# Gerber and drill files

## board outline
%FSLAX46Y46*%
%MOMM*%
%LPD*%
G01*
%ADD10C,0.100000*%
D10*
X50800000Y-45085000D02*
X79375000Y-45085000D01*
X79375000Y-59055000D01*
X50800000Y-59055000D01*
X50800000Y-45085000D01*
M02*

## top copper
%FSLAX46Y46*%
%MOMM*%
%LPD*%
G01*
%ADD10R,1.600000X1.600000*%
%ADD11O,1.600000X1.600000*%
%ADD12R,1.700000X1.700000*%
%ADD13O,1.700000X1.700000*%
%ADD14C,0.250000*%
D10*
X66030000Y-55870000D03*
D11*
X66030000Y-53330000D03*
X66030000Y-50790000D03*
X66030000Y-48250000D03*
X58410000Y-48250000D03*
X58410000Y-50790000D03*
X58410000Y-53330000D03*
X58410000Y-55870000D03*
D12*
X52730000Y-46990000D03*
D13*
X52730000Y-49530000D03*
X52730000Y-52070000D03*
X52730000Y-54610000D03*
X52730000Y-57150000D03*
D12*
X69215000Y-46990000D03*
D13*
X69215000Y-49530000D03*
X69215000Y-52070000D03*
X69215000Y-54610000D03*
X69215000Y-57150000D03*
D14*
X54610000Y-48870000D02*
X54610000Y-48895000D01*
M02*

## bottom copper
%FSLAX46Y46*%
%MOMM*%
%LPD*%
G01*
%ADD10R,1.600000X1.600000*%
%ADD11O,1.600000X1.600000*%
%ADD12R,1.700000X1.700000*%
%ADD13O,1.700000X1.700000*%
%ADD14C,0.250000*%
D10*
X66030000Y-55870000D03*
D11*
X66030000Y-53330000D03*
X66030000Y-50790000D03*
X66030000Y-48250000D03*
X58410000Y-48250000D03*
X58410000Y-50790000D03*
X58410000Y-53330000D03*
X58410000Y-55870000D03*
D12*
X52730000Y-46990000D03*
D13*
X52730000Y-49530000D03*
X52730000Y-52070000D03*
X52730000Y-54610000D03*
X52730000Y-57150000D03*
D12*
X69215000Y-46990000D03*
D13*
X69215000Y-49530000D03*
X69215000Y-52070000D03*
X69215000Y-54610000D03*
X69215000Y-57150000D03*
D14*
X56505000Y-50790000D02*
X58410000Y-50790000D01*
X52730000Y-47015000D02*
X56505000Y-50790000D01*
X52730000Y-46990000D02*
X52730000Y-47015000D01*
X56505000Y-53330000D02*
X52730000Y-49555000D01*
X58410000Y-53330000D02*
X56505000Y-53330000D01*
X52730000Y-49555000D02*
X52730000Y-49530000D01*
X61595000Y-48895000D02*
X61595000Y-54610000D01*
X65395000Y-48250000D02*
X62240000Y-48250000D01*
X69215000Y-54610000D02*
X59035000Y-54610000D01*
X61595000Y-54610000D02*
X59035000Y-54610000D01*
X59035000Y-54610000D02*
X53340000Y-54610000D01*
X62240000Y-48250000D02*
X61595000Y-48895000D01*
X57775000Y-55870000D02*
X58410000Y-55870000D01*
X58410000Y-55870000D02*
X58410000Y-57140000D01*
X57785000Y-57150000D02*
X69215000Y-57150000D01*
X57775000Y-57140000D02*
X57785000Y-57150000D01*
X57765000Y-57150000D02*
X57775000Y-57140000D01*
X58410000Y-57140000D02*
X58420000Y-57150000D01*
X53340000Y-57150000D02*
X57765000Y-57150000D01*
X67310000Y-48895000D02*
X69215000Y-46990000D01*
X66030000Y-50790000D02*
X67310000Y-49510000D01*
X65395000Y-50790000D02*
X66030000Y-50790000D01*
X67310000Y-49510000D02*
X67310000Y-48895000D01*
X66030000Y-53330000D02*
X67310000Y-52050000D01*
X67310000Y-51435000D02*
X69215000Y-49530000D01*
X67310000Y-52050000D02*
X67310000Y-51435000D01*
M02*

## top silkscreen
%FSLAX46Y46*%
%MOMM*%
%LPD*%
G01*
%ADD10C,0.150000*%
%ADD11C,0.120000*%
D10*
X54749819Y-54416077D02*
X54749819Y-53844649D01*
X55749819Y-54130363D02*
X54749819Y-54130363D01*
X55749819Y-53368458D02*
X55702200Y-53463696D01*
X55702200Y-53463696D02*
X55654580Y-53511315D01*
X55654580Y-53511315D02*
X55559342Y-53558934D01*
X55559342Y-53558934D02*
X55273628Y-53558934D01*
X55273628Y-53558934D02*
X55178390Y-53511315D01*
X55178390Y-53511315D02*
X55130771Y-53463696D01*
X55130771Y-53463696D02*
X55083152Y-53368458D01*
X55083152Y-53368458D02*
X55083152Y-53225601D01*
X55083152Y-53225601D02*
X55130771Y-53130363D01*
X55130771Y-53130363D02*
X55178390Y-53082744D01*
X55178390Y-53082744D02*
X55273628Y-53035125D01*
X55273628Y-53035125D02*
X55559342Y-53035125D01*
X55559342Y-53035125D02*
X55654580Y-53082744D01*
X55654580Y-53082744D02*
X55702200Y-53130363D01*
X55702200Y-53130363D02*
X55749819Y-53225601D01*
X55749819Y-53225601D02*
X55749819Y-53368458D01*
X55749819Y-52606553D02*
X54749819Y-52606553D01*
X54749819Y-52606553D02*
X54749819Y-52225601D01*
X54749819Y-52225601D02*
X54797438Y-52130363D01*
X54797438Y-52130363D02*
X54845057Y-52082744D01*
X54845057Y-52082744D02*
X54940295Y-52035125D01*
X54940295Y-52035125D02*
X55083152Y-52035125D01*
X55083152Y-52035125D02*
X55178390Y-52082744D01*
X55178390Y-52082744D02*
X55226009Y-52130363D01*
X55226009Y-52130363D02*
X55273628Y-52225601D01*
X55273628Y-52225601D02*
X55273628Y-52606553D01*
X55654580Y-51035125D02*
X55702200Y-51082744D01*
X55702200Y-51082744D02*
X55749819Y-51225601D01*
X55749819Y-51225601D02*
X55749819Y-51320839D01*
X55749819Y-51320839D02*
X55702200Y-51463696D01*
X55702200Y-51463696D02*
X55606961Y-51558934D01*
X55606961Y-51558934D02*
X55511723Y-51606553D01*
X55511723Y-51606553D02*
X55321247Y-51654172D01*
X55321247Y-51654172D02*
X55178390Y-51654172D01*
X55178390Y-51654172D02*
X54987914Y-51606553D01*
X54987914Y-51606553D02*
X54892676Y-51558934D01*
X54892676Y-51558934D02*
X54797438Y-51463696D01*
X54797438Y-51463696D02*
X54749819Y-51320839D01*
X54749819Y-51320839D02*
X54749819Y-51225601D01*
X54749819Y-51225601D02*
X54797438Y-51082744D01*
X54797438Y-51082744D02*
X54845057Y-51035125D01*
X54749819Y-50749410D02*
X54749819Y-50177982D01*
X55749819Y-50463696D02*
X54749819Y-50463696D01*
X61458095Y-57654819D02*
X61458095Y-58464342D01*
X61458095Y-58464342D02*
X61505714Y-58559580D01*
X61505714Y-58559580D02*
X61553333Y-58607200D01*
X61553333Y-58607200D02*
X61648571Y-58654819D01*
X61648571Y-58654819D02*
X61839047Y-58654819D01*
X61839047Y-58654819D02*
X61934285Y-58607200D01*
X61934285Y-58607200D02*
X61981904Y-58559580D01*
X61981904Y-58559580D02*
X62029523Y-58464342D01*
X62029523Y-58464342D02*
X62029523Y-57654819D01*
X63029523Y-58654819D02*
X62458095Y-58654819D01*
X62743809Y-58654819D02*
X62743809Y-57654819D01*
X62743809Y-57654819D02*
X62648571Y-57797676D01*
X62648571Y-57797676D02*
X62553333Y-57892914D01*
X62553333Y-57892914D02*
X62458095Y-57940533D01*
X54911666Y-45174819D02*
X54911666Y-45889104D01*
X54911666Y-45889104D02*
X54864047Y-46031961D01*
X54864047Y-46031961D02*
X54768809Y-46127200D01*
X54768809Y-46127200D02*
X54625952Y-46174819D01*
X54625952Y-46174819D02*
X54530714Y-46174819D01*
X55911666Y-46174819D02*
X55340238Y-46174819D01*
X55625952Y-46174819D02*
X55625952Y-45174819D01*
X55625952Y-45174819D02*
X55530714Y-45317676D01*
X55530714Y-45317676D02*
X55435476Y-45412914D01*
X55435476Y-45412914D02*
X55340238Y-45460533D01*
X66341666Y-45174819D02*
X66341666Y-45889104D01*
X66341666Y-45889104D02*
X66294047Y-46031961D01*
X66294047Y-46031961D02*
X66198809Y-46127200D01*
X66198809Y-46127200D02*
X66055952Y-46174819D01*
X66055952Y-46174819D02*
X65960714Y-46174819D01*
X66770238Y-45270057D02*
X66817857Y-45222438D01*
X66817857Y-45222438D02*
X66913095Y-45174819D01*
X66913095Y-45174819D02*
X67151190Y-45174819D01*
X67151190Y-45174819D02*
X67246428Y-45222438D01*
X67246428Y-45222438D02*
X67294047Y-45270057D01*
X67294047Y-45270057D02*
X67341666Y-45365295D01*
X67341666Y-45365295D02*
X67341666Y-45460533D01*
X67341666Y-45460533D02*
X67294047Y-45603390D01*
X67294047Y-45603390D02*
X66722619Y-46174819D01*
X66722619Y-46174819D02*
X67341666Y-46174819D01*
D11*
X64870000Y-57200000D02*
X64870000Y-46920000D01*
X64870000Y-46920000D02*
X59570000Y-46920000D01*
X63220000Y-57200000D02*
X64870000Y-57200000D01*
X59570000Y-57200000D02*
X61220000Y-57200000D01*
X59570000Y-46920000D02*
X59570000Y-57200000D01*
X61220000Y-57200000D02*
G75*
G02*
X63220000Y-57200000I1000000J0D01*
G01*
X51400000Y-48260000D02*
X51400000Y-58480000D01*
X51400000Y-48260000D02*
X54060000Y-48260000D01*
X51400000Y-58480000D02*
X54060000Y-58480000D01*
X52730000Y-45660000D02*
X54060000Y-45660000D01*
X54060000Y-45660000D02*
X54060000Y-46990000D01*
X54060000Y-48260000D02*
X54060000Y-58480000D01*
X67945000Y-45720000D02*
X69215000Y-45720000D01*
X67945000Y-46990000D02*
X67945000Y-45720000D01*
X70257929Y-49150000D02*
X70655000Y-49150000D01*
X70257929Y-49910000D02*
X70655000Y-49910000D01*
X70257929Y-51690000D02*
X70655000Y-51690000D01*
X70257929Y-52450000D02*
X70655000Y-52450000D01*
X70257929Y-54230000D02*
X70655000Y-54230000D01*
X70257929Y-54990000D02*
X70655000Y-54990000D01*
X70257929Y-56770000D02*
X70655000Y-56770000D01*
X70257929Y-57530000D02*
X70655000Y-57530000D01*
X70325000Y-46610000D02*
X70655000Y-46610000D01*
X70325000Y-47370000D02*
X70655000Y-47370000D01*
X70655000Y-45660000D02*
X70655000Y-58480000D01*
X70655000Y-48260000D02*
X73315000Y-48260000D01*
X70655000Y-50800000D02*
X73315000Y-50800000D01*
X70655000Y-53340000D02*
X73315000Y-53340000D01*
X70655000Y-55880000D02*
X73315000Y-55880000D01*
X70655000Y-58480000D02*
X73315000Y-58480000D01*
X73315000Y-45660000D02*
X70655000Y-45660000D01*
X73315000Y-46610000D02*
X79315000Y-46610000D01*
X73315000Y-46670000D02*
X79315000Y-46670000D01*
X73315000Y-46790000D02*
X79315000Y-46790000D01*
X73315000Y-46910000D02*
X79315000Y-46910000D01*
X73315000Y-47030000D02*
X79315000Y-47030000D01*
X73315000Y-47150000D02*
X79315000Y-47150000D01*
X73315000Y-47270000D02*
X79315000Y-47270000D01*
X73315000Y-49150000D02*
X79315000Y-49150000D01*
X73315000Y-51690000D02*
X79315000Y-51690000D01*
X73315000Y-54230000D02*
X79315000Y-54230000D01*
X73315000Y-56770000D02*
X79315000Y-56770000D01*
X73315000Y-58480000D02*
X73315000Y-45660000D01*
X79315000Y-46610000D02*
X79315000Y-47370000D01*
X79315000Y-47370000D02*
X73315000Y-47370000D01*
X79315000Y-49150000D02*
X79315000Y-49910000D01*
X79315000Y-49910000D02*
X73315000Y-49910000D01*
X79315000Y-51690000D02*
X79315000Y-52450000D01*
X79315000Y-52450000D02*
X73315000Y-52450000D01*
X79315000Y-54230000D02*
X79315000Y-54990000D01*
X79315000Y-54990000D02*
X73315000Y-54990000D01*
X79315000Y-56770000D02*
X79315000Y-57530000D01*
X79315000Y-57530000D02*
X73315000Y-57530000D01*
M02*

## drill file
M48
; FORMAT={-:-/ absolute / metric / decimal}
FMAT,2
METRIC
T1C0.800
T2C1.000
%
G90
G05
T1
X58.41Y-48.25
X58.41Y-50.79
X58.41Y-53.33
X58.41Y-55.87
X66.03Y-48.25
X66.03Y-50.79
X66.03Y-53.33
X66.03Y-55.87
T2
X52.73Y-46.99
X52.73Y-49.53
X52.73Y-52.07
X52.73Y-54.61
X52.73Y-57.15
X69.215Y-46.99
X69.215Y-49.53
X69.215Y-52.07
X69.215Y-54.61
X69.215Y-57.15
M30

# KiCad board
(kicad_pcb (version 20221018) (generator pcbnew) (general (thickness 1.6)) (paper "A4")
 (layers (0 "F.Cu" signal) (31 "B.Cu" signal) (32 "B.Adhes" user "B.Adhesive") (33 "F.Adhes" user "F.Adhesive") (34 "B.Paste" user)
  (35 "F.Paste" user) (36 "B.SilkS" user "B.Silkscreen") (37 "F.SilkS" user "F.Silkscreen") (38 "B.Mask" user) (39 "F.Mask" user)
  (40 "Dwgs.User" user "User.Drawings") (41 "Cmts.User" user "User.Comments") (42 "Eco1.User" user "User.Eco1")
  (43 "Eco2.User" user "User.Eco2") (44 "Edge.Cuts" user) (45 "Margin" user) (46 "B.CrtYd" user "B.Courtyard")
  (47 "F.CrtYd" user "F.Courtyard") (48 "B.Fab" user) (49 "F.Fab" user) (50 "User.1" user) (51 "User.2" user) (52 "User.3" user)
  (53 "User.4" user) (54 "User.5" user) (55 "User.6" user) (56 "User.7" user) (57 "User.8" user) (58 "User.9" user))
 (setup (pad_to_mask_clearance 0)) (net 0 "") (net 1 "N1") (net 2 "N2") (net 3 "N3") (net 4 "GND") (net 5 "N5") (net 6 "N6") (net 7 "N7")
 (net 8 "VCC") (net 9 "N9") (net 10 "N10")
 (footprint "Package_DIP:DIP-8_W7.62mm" (layer "F.Cu") (at 66.03 55.87 180)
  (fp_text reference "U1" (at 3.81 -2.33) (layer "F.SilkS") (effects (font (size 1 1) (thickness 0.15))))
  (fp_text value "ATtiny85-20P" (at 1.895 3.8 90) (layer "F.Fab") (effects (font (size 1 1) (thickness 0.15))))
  (fp_line (start 1.16 -1.33) (end 1.16 8.95) (stroke (width 0.12) (type solid)) (layer "F.SilkS"))
  (fp_line (start 1.16 8.95) (end 6.46 8.95) (stroke (width 0.12) (type solid)) (layer "F.SilkS"))
  (fp_line (start 2.81 -1.33) (end 1.16 -1.33) (stroke (width 0.12) (type solid)) (layer "F.SilkS"))
  (fp_line (start 6.46 -1.33) (end 4.81 -1.33) (stroke (width 0.12) (type solid)) (layer "F.SilkS"))
  (fp_line (start 6.46 8.95) (end 6.46 -1.33) (stroke (width 0.12) (type solid)) (layer "F.SilkS"))
  (fp_arc (start 4.81 -1.33) (mid 3.81 -0.33) (end 2.81 -1.33) (stroke (width 0.12) (type solid)) (layer "F.SilkS"))
  (pad "1" thru_hole rect (at 0 0 180) (size 1.6 1.6) (drill 0.8) (layers "*.Cu" "*.Mask") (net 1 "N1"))
  (pad "2" thru_hole oval (at 0 2.54 180) (size 1.6 1.6) (drill 0.8) (layers "*.Cu" "*.Mask") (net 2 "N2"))
  (pad "3" thru_hole oval (at 0 5.08 180) (size 1.6 1.6) (drill 0.8) (layers "*.Cu" "*.Mask") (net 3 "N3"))
  (pad "4" thru_hole oval (at 0 7.62 180) (size 1.6 1.6) (drill 0.8) (layers "*.Cu" "*.Mask") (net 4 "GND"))
  (pad "5" thru_hole oval (at 7.62 7.62 180) (size 1.6 1.6) (drill 0.8) (layers "*.Cu" "*.Mask") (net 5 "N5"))
  (pad "6" thru_hole oval (at 7.62 5.08 180) (size 1.6 1.6) (drill 0.8) (layers "*.Cu" "*.Mask") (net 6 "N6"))
  (pad "7" thru_hole oval (at 7.62 2.54 180) (size 1.6 1.6) (drill 0.8) (layers "*.Cu" "*.Mask") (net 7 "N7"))
  (pad "8" thru_hole oval (at 7.62 0 180) (size 1.6 1.6) (drill 0.8) (layers "*.Cu" "*.Mask") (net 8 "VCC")))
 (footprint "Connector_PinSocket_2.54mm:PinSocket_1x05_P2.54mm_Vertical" (layer "F.Cu") (at 52.73 46.99)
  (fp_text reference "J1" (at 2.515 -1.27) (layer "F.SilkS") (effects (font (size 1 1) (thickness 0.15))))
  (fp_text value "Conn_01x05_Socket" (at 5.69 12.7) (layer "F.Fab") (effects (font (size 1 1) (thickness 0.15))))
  (fp_line (start -1.33 1.27) (end -1.33 11.49) (stroke (width 0.12) (type solid)) (layer "F.SilkS"))
  (fp_line (start -1.33 1.27) (end 1.33 1.27) (stroke (width 0.12) (type solid)) (layer "F.SilkS"))
  (fp_line (start -1.33 11.49) (end 1.33 11.49) (stroke (width 0.12) (type solid)) (layer "F.SilkS"))
  (fp_line (start 0 -1.33) (end 1.33 -1.33) (stroke (width 0.12) (type solid)) (layer "F.SilkS"))
  (fp_line (start 1.33 -1.33) (end 1.33 0) (stroke (width 0.12) (type solid)) (layer "F.SilkS"))
  (fp_line (start 1.33 1.27) (end 1.33 11.49) (stroke (width 0.12) (type solid)) (layer "F.SilkS"))
  (pad "1" thru_hole rect (at 0 0) (size 1.7 1.7) (drill 1) (layers "*.Cu" "*.Mask") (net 6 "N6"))
  (pad "2" thru_hole oval (at 0 2.54) (size 1.7 1.7) (drill 1) (layers "*.Cu" "*.Mask") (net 7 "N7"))
  (pad "3" thru_hole oval (at 0 5.08) (size 1.7 1.7) (drill 1) (layers "*.Cu" "*.Mask") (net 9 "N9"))
  (pad "4" thru_hole oval (at 0 7.62) (size 1.7 1.7) (drill 1) (layers "*.Cu" "*.Mask") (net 4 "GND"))
  (pad "5" thru_hole oval (at 0 10.16) (size 1.7 1.7) (drill 1) (layers "*.Cu" "*.Mask") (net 8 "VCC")))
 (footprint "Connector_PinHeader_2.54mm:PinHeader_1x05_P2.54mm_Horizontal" (layer "F.Cu") (at 69.215 46.99)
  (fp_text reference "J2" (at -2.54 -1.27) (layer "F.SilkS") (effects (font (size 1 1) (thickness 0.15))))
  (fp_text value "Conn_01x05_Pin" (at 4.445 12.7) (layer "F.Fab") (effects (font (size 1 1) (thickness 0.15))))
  (fp_line (start -1.27 -1.27) (end 0 -1.27) (stroke (width 0.12) (type solid)) (layer "F.SilkS"))
  (fp_line (start -1.27 0) (end -1.27 -1.27) (stroke (width 0.12) (type solid)) (layer "F.SilkS"))
  (fp_line (start 1.042929 2.16) (end 1.44 2.16) (stroke (width 0.12) (type solid)) (layer "F.SilkS"))
  (fp_line (start 1.042929 2.92) (end 1.44 2.92) (stroke (width 0.12) (type solid)) (layer "F.SilkS"))
  (fp_line (start 1.042929 4.7) (end 1.44 4.7) (stroke (width 0.12) (type solid)) (layer "F.SilkS"))
  (fp_line (start 1.042929 5.46) (end 1.44 5.46) (stroke (width 0.12) (type solid)) (layer "F.SilkS"))
  (fp_line (start 1.042929 7.24) (end 1.44 7.24) (stroke (width 0.12) (type solid)) (layer "F.SilkS"))
  (fp_line (start 1.042929 8) (end 1.44 8) (stroke (width 0.12) (type solid)) (layer "F.SilkS"))
  (fp_line (start 1.042929 9.78) (end 1.44 9.78) (stroke (width 0.12) (type solid)) (layer "F.SilkS"))
  (fp_line (start 1.042929 10.54) (end 1.44 10.54) (stroke (width 0.12) (type solid)) (layer "F.SilkS"))
  (fp_line (start 1.11 -0.38) (end 1.44 -0.38) (stroke (width 0.12) (type solid)) (layer "F.SilkS"))
  (fp_line (start 1.11 0.38) (end 1.44 0.38) (stroke (width 0.12) (type solid)) (layer "F.SilkS"))
  (fp_line (start 1.44 -1.33) (end 1.44 11.49) (stroke (width 0.12) (type solid)) (layer "F.SilkS"))
  (fp_line (start 1.44 1.27) (end 4.1 1.27) (stroke (width 0.12) (type solid)) (layer "F.SilkS"))
  (fp_line (start 1.44 3.81) (end 4.1 3.81) (stroke (width 0.12) (type solid)) (layer "F.SilkS"))
  (fp_line (start 1.44 6.35) (end 4.1 6.35) (stroke (width 0.12) (type solid)) (layer "F.SilkS"))
  (fp_line (start 1.44 8.89) (end 4.1 8.89) (stroke (width 0.12) (type solid)) (layer "F.SilkS"))
  (fp_line (start 1.44 11.49) (end 4.1 11.49) (stroke (width 0.12) (type solid)) (layer "F.SilkS"))
  (fp_line (start 4.1 -1.33) (end 1.44 -1.33) (stroke (width 0.12) (type solid)) (layer "F.SilkS"))
  (fp_line (start 4.1 -0.38) (end 10.1 -0.38) (stroke (width 0.12) (type solid)) (layer "F.SilkS"))
  (fp_line (start 4.1 -0.32) (end 10.1 -0.32) (stroke (width 0.12) (type solid)) (layer "F.SilkS"))
  (fp_line (start 4.1 -0.2) (end 10.1 -0.2) (stroke (width 0.12) (type solid)) (layer "F.SilkS"))
  (fp_line (start 4.1 -0.08) (end 10.1 -0.08) (stroke (width 0.12) (type solid)) (layer "F.SilkS"))
  (fp_line (start 4.1 0.04) (end 10.1 0.04) (stroke (width 0.12) (type solid)) (layer "F.SilkS"))
  (fp_line (start 4.1 0.16) (end 10.1 0.16) (stroke (width 0.12) (type solid)) (layer "F.SilkS"))
  (fp_line (start 4.1 0.28) (end 10.1 0.28) (stroke (width 0.12) (type solid)) (layer "F.SilkS"))
  (fp_line (start 4.1 2.16) (end 10.1 2.16) (stroke (width 0.12) (type solid)) (layer "F.SilkS"))
  (fp_line (start 4.1 4.7) (end 10.1 4.7) (stroke (width 0.12) (type solid)) (layer "F.SilkS"))
  (fp_line (start 4.1 7.24) (end 10.1 7.24) (stroke (width 0.12) (type solid)) (layer "F.SilkS"))
  (fp_line (start 4.1 9.78) (end 10.1 9.78) (stroke (width 0.12) (type solid)) (layer "F.SilkS"))
  (fp_line (start 4.1 11.49) (end 4.1 -1.33) (stroke (width 0.12) (type solid)) (layer "F.SilkS"))
  (fp_line (start 10.1 -0.38) (end 10.1 0.38) (stroke (width 0.12) (type solid)) (layer "F.SilkS"))
  (fp_line (start 10.1 0.38) (end 4.1 0.38) (stroke (width 0.12) (type solid)) (layer "F.SilkS"))
  (fp_line (start 10.1 2.16) (end 10.1 2.92) (stroke (width 0.12) (type solid)) (layer "F.SilkS"))
  (fp_line (start 10.1 2.92) (end 4.1 2.92) (stroke (width 0.12) (type solid)) (layer "F.SilkS"))
  (fp_line (start 10.1 4.7) (end 10.1 5.46) (stroke (width 0.12) (type solid)) (layer "F.SilkS"))
  (fp_line (start 10.1 5.46) (end 4.1 5.46) (stroke (width 0.12) (type solid)) (layer "F.SilkS"))
  (fp_line (start 10.1 7.24) (end 10.1 8) (stroke (width 0.12) (type solid)) (layer "F.SilkS"))
  (fp_line (start 10.1 8) (end 4.1 8) (stroke (width 0.12) (type solid)) (layer "F.SilkS"))
  (fp_line (start 10.1 9.78) (end 10.1 10.54) (stroke (width 0.12) (type solid)) (layer "F.SilkS"))
  (fp_line (start 10.1 10.54) (end 4.1 10.54) (stroke (width 0.12) (type solid)) (layer "F.SilkS"))
  (pad "1" thru_hole rect (at 0 0) (size 1.7 1.7) (drill 1) (layers "*.Cu" "*.Mask") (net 3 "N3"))
  (pad "2" thru_hole oval (at 0 2.54) (size 1.7 1.7) (drill 1) (layers "*.Cu" "*.Mask") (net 2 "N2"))
  (pad "3" thru_hole oval (at 0 5.08) (size 1.7 1.7) (drill 1) (layers "*.Cu" "*.Mask") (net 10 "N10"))
  (pad "4" thru_hole oval (at 0 7.62) (size 1.7 1.7) (drill 1) (layers "*.Cu" "*.Mask") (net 4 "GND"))
  (pad "5" thru_hole oval (at 0 10.16) (size 1.7 1.7) (drill 1) (layers "*.Cu" "*.Mask") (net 8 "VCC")))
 (gr_rect (start 50.8 45.085) (end 79.375 59.055) (stroke (width 0.1) (type default)) (fill none) (layer "Edge.Cuts"))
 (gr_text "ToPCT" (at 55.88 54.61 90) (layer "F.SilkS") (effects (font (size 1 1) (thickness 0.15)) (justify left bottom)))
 (segment (start 54.61 48.87) (end 54.61 48.895) (width 0.25) (layer "F.Cu") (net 6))
 (segment (start 56.505 50.79) (end 58.41 50.79) (width 0.25) (layer "B.Cu") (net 6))
 (segment (start 52.73 47.015) (end 56.505 50.79) (width 0.25) (layer "B.Cu") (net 6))
 (segment (start 52.73 46.99) (end 52.73 47.015) (width 0.25) (layer "B.Cu") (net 6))
 (segment (start 56.505 53.33) (end 52.73 49.555) (width 0.25) (layer "B.Cu") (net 7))
 (segment (start 58.41 53.33) (end 56.505 53.33) (width 0.25) (layer "B.Cu") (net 7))
 (segment (start 52.73 49.555) (end 52.73 49.53) (width 0.25) (layer "B.Cu") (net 7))
 (segment (start 61.595 48.895) (end 61.595 54.61) (width 0.25) (layer "B.Cu") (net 4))
 (segment (start 65.395 48.25) (end 62.24 48.25) (width 0.25) (layer "B.Cu") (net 4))
 (segment (start 69.215 54.61) (end 59.035 54.61) (width 0.25) (layer "B.Cu") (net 4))
 (segment (start 61.595 54.61) (end 59.035 54.61) (width 0.25) (layer "B.Cu") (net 4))
 (segment (start 59.035 54.61) (end 53.34 54.61) (width 0.25) (layer "B.Cu") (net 4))
 (segment (start 62.24 48.25) (end 61.595 48.895) (width 0.25) (layer "B.Cu") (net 4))
 (segment (start 57.775 55.87) (end 58.41 55.87) (width 0.25) (layer "B.Cu") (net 8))
 (segment (start 58.41 55.87) (end 58.41 57.14) (width 0.25) (layer "B.Cu") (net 8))
 (segment (start 57.785 57.15) (end 69.215 57.15) (width 0.25) (layer "B.Cu") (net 8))
 (segment (start 57.775 57.14) (end 57.785 57.15) (width 0.25) (layer "B.Cu") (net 8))
 (segment (start 57.765 57.15) (end 57.775 57.14) (width 0.25) (layer "B.Cu") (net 8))
 (segment (start 58.41 57.14) (end 58.42 57.15) (width 0.25) (layer "B.Cu") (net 8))
 (segment (start 53.34 57.15) (end 57.765 57.15) (width 0.25) (layer "B.Cu") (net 8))
 (segment (start 67.31 48.895) (end 69.215 46.99) (width 0.25) (layer "B.Cu") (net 3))
 (segment (start 66.03 50.79) (end 67.31 49.51) (width 0.25) (layer "B.Cu") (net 3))
 (segment (start 65.395 50.79) (end 66.03 50.79) (width 0.25) (layer "B.Cu") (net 3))
 (segment (start 67.31 49.51) (end 67.31 48.895) (width 0.25) (layer "B.Cu") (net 3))
 (segment (start 66.03 53.33) (end 67.31 52.05) (width 0.25) (layer "B.Cu") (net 2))
 (segment (start 67.31 51.435) (end 69.215 49.53) (width 0.25) (layer "B.Cu") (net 2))
 (segment (start 67.31 52.05) (end 67.31 51.435) (width 0.25) (layer "B.Cu") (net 2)))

